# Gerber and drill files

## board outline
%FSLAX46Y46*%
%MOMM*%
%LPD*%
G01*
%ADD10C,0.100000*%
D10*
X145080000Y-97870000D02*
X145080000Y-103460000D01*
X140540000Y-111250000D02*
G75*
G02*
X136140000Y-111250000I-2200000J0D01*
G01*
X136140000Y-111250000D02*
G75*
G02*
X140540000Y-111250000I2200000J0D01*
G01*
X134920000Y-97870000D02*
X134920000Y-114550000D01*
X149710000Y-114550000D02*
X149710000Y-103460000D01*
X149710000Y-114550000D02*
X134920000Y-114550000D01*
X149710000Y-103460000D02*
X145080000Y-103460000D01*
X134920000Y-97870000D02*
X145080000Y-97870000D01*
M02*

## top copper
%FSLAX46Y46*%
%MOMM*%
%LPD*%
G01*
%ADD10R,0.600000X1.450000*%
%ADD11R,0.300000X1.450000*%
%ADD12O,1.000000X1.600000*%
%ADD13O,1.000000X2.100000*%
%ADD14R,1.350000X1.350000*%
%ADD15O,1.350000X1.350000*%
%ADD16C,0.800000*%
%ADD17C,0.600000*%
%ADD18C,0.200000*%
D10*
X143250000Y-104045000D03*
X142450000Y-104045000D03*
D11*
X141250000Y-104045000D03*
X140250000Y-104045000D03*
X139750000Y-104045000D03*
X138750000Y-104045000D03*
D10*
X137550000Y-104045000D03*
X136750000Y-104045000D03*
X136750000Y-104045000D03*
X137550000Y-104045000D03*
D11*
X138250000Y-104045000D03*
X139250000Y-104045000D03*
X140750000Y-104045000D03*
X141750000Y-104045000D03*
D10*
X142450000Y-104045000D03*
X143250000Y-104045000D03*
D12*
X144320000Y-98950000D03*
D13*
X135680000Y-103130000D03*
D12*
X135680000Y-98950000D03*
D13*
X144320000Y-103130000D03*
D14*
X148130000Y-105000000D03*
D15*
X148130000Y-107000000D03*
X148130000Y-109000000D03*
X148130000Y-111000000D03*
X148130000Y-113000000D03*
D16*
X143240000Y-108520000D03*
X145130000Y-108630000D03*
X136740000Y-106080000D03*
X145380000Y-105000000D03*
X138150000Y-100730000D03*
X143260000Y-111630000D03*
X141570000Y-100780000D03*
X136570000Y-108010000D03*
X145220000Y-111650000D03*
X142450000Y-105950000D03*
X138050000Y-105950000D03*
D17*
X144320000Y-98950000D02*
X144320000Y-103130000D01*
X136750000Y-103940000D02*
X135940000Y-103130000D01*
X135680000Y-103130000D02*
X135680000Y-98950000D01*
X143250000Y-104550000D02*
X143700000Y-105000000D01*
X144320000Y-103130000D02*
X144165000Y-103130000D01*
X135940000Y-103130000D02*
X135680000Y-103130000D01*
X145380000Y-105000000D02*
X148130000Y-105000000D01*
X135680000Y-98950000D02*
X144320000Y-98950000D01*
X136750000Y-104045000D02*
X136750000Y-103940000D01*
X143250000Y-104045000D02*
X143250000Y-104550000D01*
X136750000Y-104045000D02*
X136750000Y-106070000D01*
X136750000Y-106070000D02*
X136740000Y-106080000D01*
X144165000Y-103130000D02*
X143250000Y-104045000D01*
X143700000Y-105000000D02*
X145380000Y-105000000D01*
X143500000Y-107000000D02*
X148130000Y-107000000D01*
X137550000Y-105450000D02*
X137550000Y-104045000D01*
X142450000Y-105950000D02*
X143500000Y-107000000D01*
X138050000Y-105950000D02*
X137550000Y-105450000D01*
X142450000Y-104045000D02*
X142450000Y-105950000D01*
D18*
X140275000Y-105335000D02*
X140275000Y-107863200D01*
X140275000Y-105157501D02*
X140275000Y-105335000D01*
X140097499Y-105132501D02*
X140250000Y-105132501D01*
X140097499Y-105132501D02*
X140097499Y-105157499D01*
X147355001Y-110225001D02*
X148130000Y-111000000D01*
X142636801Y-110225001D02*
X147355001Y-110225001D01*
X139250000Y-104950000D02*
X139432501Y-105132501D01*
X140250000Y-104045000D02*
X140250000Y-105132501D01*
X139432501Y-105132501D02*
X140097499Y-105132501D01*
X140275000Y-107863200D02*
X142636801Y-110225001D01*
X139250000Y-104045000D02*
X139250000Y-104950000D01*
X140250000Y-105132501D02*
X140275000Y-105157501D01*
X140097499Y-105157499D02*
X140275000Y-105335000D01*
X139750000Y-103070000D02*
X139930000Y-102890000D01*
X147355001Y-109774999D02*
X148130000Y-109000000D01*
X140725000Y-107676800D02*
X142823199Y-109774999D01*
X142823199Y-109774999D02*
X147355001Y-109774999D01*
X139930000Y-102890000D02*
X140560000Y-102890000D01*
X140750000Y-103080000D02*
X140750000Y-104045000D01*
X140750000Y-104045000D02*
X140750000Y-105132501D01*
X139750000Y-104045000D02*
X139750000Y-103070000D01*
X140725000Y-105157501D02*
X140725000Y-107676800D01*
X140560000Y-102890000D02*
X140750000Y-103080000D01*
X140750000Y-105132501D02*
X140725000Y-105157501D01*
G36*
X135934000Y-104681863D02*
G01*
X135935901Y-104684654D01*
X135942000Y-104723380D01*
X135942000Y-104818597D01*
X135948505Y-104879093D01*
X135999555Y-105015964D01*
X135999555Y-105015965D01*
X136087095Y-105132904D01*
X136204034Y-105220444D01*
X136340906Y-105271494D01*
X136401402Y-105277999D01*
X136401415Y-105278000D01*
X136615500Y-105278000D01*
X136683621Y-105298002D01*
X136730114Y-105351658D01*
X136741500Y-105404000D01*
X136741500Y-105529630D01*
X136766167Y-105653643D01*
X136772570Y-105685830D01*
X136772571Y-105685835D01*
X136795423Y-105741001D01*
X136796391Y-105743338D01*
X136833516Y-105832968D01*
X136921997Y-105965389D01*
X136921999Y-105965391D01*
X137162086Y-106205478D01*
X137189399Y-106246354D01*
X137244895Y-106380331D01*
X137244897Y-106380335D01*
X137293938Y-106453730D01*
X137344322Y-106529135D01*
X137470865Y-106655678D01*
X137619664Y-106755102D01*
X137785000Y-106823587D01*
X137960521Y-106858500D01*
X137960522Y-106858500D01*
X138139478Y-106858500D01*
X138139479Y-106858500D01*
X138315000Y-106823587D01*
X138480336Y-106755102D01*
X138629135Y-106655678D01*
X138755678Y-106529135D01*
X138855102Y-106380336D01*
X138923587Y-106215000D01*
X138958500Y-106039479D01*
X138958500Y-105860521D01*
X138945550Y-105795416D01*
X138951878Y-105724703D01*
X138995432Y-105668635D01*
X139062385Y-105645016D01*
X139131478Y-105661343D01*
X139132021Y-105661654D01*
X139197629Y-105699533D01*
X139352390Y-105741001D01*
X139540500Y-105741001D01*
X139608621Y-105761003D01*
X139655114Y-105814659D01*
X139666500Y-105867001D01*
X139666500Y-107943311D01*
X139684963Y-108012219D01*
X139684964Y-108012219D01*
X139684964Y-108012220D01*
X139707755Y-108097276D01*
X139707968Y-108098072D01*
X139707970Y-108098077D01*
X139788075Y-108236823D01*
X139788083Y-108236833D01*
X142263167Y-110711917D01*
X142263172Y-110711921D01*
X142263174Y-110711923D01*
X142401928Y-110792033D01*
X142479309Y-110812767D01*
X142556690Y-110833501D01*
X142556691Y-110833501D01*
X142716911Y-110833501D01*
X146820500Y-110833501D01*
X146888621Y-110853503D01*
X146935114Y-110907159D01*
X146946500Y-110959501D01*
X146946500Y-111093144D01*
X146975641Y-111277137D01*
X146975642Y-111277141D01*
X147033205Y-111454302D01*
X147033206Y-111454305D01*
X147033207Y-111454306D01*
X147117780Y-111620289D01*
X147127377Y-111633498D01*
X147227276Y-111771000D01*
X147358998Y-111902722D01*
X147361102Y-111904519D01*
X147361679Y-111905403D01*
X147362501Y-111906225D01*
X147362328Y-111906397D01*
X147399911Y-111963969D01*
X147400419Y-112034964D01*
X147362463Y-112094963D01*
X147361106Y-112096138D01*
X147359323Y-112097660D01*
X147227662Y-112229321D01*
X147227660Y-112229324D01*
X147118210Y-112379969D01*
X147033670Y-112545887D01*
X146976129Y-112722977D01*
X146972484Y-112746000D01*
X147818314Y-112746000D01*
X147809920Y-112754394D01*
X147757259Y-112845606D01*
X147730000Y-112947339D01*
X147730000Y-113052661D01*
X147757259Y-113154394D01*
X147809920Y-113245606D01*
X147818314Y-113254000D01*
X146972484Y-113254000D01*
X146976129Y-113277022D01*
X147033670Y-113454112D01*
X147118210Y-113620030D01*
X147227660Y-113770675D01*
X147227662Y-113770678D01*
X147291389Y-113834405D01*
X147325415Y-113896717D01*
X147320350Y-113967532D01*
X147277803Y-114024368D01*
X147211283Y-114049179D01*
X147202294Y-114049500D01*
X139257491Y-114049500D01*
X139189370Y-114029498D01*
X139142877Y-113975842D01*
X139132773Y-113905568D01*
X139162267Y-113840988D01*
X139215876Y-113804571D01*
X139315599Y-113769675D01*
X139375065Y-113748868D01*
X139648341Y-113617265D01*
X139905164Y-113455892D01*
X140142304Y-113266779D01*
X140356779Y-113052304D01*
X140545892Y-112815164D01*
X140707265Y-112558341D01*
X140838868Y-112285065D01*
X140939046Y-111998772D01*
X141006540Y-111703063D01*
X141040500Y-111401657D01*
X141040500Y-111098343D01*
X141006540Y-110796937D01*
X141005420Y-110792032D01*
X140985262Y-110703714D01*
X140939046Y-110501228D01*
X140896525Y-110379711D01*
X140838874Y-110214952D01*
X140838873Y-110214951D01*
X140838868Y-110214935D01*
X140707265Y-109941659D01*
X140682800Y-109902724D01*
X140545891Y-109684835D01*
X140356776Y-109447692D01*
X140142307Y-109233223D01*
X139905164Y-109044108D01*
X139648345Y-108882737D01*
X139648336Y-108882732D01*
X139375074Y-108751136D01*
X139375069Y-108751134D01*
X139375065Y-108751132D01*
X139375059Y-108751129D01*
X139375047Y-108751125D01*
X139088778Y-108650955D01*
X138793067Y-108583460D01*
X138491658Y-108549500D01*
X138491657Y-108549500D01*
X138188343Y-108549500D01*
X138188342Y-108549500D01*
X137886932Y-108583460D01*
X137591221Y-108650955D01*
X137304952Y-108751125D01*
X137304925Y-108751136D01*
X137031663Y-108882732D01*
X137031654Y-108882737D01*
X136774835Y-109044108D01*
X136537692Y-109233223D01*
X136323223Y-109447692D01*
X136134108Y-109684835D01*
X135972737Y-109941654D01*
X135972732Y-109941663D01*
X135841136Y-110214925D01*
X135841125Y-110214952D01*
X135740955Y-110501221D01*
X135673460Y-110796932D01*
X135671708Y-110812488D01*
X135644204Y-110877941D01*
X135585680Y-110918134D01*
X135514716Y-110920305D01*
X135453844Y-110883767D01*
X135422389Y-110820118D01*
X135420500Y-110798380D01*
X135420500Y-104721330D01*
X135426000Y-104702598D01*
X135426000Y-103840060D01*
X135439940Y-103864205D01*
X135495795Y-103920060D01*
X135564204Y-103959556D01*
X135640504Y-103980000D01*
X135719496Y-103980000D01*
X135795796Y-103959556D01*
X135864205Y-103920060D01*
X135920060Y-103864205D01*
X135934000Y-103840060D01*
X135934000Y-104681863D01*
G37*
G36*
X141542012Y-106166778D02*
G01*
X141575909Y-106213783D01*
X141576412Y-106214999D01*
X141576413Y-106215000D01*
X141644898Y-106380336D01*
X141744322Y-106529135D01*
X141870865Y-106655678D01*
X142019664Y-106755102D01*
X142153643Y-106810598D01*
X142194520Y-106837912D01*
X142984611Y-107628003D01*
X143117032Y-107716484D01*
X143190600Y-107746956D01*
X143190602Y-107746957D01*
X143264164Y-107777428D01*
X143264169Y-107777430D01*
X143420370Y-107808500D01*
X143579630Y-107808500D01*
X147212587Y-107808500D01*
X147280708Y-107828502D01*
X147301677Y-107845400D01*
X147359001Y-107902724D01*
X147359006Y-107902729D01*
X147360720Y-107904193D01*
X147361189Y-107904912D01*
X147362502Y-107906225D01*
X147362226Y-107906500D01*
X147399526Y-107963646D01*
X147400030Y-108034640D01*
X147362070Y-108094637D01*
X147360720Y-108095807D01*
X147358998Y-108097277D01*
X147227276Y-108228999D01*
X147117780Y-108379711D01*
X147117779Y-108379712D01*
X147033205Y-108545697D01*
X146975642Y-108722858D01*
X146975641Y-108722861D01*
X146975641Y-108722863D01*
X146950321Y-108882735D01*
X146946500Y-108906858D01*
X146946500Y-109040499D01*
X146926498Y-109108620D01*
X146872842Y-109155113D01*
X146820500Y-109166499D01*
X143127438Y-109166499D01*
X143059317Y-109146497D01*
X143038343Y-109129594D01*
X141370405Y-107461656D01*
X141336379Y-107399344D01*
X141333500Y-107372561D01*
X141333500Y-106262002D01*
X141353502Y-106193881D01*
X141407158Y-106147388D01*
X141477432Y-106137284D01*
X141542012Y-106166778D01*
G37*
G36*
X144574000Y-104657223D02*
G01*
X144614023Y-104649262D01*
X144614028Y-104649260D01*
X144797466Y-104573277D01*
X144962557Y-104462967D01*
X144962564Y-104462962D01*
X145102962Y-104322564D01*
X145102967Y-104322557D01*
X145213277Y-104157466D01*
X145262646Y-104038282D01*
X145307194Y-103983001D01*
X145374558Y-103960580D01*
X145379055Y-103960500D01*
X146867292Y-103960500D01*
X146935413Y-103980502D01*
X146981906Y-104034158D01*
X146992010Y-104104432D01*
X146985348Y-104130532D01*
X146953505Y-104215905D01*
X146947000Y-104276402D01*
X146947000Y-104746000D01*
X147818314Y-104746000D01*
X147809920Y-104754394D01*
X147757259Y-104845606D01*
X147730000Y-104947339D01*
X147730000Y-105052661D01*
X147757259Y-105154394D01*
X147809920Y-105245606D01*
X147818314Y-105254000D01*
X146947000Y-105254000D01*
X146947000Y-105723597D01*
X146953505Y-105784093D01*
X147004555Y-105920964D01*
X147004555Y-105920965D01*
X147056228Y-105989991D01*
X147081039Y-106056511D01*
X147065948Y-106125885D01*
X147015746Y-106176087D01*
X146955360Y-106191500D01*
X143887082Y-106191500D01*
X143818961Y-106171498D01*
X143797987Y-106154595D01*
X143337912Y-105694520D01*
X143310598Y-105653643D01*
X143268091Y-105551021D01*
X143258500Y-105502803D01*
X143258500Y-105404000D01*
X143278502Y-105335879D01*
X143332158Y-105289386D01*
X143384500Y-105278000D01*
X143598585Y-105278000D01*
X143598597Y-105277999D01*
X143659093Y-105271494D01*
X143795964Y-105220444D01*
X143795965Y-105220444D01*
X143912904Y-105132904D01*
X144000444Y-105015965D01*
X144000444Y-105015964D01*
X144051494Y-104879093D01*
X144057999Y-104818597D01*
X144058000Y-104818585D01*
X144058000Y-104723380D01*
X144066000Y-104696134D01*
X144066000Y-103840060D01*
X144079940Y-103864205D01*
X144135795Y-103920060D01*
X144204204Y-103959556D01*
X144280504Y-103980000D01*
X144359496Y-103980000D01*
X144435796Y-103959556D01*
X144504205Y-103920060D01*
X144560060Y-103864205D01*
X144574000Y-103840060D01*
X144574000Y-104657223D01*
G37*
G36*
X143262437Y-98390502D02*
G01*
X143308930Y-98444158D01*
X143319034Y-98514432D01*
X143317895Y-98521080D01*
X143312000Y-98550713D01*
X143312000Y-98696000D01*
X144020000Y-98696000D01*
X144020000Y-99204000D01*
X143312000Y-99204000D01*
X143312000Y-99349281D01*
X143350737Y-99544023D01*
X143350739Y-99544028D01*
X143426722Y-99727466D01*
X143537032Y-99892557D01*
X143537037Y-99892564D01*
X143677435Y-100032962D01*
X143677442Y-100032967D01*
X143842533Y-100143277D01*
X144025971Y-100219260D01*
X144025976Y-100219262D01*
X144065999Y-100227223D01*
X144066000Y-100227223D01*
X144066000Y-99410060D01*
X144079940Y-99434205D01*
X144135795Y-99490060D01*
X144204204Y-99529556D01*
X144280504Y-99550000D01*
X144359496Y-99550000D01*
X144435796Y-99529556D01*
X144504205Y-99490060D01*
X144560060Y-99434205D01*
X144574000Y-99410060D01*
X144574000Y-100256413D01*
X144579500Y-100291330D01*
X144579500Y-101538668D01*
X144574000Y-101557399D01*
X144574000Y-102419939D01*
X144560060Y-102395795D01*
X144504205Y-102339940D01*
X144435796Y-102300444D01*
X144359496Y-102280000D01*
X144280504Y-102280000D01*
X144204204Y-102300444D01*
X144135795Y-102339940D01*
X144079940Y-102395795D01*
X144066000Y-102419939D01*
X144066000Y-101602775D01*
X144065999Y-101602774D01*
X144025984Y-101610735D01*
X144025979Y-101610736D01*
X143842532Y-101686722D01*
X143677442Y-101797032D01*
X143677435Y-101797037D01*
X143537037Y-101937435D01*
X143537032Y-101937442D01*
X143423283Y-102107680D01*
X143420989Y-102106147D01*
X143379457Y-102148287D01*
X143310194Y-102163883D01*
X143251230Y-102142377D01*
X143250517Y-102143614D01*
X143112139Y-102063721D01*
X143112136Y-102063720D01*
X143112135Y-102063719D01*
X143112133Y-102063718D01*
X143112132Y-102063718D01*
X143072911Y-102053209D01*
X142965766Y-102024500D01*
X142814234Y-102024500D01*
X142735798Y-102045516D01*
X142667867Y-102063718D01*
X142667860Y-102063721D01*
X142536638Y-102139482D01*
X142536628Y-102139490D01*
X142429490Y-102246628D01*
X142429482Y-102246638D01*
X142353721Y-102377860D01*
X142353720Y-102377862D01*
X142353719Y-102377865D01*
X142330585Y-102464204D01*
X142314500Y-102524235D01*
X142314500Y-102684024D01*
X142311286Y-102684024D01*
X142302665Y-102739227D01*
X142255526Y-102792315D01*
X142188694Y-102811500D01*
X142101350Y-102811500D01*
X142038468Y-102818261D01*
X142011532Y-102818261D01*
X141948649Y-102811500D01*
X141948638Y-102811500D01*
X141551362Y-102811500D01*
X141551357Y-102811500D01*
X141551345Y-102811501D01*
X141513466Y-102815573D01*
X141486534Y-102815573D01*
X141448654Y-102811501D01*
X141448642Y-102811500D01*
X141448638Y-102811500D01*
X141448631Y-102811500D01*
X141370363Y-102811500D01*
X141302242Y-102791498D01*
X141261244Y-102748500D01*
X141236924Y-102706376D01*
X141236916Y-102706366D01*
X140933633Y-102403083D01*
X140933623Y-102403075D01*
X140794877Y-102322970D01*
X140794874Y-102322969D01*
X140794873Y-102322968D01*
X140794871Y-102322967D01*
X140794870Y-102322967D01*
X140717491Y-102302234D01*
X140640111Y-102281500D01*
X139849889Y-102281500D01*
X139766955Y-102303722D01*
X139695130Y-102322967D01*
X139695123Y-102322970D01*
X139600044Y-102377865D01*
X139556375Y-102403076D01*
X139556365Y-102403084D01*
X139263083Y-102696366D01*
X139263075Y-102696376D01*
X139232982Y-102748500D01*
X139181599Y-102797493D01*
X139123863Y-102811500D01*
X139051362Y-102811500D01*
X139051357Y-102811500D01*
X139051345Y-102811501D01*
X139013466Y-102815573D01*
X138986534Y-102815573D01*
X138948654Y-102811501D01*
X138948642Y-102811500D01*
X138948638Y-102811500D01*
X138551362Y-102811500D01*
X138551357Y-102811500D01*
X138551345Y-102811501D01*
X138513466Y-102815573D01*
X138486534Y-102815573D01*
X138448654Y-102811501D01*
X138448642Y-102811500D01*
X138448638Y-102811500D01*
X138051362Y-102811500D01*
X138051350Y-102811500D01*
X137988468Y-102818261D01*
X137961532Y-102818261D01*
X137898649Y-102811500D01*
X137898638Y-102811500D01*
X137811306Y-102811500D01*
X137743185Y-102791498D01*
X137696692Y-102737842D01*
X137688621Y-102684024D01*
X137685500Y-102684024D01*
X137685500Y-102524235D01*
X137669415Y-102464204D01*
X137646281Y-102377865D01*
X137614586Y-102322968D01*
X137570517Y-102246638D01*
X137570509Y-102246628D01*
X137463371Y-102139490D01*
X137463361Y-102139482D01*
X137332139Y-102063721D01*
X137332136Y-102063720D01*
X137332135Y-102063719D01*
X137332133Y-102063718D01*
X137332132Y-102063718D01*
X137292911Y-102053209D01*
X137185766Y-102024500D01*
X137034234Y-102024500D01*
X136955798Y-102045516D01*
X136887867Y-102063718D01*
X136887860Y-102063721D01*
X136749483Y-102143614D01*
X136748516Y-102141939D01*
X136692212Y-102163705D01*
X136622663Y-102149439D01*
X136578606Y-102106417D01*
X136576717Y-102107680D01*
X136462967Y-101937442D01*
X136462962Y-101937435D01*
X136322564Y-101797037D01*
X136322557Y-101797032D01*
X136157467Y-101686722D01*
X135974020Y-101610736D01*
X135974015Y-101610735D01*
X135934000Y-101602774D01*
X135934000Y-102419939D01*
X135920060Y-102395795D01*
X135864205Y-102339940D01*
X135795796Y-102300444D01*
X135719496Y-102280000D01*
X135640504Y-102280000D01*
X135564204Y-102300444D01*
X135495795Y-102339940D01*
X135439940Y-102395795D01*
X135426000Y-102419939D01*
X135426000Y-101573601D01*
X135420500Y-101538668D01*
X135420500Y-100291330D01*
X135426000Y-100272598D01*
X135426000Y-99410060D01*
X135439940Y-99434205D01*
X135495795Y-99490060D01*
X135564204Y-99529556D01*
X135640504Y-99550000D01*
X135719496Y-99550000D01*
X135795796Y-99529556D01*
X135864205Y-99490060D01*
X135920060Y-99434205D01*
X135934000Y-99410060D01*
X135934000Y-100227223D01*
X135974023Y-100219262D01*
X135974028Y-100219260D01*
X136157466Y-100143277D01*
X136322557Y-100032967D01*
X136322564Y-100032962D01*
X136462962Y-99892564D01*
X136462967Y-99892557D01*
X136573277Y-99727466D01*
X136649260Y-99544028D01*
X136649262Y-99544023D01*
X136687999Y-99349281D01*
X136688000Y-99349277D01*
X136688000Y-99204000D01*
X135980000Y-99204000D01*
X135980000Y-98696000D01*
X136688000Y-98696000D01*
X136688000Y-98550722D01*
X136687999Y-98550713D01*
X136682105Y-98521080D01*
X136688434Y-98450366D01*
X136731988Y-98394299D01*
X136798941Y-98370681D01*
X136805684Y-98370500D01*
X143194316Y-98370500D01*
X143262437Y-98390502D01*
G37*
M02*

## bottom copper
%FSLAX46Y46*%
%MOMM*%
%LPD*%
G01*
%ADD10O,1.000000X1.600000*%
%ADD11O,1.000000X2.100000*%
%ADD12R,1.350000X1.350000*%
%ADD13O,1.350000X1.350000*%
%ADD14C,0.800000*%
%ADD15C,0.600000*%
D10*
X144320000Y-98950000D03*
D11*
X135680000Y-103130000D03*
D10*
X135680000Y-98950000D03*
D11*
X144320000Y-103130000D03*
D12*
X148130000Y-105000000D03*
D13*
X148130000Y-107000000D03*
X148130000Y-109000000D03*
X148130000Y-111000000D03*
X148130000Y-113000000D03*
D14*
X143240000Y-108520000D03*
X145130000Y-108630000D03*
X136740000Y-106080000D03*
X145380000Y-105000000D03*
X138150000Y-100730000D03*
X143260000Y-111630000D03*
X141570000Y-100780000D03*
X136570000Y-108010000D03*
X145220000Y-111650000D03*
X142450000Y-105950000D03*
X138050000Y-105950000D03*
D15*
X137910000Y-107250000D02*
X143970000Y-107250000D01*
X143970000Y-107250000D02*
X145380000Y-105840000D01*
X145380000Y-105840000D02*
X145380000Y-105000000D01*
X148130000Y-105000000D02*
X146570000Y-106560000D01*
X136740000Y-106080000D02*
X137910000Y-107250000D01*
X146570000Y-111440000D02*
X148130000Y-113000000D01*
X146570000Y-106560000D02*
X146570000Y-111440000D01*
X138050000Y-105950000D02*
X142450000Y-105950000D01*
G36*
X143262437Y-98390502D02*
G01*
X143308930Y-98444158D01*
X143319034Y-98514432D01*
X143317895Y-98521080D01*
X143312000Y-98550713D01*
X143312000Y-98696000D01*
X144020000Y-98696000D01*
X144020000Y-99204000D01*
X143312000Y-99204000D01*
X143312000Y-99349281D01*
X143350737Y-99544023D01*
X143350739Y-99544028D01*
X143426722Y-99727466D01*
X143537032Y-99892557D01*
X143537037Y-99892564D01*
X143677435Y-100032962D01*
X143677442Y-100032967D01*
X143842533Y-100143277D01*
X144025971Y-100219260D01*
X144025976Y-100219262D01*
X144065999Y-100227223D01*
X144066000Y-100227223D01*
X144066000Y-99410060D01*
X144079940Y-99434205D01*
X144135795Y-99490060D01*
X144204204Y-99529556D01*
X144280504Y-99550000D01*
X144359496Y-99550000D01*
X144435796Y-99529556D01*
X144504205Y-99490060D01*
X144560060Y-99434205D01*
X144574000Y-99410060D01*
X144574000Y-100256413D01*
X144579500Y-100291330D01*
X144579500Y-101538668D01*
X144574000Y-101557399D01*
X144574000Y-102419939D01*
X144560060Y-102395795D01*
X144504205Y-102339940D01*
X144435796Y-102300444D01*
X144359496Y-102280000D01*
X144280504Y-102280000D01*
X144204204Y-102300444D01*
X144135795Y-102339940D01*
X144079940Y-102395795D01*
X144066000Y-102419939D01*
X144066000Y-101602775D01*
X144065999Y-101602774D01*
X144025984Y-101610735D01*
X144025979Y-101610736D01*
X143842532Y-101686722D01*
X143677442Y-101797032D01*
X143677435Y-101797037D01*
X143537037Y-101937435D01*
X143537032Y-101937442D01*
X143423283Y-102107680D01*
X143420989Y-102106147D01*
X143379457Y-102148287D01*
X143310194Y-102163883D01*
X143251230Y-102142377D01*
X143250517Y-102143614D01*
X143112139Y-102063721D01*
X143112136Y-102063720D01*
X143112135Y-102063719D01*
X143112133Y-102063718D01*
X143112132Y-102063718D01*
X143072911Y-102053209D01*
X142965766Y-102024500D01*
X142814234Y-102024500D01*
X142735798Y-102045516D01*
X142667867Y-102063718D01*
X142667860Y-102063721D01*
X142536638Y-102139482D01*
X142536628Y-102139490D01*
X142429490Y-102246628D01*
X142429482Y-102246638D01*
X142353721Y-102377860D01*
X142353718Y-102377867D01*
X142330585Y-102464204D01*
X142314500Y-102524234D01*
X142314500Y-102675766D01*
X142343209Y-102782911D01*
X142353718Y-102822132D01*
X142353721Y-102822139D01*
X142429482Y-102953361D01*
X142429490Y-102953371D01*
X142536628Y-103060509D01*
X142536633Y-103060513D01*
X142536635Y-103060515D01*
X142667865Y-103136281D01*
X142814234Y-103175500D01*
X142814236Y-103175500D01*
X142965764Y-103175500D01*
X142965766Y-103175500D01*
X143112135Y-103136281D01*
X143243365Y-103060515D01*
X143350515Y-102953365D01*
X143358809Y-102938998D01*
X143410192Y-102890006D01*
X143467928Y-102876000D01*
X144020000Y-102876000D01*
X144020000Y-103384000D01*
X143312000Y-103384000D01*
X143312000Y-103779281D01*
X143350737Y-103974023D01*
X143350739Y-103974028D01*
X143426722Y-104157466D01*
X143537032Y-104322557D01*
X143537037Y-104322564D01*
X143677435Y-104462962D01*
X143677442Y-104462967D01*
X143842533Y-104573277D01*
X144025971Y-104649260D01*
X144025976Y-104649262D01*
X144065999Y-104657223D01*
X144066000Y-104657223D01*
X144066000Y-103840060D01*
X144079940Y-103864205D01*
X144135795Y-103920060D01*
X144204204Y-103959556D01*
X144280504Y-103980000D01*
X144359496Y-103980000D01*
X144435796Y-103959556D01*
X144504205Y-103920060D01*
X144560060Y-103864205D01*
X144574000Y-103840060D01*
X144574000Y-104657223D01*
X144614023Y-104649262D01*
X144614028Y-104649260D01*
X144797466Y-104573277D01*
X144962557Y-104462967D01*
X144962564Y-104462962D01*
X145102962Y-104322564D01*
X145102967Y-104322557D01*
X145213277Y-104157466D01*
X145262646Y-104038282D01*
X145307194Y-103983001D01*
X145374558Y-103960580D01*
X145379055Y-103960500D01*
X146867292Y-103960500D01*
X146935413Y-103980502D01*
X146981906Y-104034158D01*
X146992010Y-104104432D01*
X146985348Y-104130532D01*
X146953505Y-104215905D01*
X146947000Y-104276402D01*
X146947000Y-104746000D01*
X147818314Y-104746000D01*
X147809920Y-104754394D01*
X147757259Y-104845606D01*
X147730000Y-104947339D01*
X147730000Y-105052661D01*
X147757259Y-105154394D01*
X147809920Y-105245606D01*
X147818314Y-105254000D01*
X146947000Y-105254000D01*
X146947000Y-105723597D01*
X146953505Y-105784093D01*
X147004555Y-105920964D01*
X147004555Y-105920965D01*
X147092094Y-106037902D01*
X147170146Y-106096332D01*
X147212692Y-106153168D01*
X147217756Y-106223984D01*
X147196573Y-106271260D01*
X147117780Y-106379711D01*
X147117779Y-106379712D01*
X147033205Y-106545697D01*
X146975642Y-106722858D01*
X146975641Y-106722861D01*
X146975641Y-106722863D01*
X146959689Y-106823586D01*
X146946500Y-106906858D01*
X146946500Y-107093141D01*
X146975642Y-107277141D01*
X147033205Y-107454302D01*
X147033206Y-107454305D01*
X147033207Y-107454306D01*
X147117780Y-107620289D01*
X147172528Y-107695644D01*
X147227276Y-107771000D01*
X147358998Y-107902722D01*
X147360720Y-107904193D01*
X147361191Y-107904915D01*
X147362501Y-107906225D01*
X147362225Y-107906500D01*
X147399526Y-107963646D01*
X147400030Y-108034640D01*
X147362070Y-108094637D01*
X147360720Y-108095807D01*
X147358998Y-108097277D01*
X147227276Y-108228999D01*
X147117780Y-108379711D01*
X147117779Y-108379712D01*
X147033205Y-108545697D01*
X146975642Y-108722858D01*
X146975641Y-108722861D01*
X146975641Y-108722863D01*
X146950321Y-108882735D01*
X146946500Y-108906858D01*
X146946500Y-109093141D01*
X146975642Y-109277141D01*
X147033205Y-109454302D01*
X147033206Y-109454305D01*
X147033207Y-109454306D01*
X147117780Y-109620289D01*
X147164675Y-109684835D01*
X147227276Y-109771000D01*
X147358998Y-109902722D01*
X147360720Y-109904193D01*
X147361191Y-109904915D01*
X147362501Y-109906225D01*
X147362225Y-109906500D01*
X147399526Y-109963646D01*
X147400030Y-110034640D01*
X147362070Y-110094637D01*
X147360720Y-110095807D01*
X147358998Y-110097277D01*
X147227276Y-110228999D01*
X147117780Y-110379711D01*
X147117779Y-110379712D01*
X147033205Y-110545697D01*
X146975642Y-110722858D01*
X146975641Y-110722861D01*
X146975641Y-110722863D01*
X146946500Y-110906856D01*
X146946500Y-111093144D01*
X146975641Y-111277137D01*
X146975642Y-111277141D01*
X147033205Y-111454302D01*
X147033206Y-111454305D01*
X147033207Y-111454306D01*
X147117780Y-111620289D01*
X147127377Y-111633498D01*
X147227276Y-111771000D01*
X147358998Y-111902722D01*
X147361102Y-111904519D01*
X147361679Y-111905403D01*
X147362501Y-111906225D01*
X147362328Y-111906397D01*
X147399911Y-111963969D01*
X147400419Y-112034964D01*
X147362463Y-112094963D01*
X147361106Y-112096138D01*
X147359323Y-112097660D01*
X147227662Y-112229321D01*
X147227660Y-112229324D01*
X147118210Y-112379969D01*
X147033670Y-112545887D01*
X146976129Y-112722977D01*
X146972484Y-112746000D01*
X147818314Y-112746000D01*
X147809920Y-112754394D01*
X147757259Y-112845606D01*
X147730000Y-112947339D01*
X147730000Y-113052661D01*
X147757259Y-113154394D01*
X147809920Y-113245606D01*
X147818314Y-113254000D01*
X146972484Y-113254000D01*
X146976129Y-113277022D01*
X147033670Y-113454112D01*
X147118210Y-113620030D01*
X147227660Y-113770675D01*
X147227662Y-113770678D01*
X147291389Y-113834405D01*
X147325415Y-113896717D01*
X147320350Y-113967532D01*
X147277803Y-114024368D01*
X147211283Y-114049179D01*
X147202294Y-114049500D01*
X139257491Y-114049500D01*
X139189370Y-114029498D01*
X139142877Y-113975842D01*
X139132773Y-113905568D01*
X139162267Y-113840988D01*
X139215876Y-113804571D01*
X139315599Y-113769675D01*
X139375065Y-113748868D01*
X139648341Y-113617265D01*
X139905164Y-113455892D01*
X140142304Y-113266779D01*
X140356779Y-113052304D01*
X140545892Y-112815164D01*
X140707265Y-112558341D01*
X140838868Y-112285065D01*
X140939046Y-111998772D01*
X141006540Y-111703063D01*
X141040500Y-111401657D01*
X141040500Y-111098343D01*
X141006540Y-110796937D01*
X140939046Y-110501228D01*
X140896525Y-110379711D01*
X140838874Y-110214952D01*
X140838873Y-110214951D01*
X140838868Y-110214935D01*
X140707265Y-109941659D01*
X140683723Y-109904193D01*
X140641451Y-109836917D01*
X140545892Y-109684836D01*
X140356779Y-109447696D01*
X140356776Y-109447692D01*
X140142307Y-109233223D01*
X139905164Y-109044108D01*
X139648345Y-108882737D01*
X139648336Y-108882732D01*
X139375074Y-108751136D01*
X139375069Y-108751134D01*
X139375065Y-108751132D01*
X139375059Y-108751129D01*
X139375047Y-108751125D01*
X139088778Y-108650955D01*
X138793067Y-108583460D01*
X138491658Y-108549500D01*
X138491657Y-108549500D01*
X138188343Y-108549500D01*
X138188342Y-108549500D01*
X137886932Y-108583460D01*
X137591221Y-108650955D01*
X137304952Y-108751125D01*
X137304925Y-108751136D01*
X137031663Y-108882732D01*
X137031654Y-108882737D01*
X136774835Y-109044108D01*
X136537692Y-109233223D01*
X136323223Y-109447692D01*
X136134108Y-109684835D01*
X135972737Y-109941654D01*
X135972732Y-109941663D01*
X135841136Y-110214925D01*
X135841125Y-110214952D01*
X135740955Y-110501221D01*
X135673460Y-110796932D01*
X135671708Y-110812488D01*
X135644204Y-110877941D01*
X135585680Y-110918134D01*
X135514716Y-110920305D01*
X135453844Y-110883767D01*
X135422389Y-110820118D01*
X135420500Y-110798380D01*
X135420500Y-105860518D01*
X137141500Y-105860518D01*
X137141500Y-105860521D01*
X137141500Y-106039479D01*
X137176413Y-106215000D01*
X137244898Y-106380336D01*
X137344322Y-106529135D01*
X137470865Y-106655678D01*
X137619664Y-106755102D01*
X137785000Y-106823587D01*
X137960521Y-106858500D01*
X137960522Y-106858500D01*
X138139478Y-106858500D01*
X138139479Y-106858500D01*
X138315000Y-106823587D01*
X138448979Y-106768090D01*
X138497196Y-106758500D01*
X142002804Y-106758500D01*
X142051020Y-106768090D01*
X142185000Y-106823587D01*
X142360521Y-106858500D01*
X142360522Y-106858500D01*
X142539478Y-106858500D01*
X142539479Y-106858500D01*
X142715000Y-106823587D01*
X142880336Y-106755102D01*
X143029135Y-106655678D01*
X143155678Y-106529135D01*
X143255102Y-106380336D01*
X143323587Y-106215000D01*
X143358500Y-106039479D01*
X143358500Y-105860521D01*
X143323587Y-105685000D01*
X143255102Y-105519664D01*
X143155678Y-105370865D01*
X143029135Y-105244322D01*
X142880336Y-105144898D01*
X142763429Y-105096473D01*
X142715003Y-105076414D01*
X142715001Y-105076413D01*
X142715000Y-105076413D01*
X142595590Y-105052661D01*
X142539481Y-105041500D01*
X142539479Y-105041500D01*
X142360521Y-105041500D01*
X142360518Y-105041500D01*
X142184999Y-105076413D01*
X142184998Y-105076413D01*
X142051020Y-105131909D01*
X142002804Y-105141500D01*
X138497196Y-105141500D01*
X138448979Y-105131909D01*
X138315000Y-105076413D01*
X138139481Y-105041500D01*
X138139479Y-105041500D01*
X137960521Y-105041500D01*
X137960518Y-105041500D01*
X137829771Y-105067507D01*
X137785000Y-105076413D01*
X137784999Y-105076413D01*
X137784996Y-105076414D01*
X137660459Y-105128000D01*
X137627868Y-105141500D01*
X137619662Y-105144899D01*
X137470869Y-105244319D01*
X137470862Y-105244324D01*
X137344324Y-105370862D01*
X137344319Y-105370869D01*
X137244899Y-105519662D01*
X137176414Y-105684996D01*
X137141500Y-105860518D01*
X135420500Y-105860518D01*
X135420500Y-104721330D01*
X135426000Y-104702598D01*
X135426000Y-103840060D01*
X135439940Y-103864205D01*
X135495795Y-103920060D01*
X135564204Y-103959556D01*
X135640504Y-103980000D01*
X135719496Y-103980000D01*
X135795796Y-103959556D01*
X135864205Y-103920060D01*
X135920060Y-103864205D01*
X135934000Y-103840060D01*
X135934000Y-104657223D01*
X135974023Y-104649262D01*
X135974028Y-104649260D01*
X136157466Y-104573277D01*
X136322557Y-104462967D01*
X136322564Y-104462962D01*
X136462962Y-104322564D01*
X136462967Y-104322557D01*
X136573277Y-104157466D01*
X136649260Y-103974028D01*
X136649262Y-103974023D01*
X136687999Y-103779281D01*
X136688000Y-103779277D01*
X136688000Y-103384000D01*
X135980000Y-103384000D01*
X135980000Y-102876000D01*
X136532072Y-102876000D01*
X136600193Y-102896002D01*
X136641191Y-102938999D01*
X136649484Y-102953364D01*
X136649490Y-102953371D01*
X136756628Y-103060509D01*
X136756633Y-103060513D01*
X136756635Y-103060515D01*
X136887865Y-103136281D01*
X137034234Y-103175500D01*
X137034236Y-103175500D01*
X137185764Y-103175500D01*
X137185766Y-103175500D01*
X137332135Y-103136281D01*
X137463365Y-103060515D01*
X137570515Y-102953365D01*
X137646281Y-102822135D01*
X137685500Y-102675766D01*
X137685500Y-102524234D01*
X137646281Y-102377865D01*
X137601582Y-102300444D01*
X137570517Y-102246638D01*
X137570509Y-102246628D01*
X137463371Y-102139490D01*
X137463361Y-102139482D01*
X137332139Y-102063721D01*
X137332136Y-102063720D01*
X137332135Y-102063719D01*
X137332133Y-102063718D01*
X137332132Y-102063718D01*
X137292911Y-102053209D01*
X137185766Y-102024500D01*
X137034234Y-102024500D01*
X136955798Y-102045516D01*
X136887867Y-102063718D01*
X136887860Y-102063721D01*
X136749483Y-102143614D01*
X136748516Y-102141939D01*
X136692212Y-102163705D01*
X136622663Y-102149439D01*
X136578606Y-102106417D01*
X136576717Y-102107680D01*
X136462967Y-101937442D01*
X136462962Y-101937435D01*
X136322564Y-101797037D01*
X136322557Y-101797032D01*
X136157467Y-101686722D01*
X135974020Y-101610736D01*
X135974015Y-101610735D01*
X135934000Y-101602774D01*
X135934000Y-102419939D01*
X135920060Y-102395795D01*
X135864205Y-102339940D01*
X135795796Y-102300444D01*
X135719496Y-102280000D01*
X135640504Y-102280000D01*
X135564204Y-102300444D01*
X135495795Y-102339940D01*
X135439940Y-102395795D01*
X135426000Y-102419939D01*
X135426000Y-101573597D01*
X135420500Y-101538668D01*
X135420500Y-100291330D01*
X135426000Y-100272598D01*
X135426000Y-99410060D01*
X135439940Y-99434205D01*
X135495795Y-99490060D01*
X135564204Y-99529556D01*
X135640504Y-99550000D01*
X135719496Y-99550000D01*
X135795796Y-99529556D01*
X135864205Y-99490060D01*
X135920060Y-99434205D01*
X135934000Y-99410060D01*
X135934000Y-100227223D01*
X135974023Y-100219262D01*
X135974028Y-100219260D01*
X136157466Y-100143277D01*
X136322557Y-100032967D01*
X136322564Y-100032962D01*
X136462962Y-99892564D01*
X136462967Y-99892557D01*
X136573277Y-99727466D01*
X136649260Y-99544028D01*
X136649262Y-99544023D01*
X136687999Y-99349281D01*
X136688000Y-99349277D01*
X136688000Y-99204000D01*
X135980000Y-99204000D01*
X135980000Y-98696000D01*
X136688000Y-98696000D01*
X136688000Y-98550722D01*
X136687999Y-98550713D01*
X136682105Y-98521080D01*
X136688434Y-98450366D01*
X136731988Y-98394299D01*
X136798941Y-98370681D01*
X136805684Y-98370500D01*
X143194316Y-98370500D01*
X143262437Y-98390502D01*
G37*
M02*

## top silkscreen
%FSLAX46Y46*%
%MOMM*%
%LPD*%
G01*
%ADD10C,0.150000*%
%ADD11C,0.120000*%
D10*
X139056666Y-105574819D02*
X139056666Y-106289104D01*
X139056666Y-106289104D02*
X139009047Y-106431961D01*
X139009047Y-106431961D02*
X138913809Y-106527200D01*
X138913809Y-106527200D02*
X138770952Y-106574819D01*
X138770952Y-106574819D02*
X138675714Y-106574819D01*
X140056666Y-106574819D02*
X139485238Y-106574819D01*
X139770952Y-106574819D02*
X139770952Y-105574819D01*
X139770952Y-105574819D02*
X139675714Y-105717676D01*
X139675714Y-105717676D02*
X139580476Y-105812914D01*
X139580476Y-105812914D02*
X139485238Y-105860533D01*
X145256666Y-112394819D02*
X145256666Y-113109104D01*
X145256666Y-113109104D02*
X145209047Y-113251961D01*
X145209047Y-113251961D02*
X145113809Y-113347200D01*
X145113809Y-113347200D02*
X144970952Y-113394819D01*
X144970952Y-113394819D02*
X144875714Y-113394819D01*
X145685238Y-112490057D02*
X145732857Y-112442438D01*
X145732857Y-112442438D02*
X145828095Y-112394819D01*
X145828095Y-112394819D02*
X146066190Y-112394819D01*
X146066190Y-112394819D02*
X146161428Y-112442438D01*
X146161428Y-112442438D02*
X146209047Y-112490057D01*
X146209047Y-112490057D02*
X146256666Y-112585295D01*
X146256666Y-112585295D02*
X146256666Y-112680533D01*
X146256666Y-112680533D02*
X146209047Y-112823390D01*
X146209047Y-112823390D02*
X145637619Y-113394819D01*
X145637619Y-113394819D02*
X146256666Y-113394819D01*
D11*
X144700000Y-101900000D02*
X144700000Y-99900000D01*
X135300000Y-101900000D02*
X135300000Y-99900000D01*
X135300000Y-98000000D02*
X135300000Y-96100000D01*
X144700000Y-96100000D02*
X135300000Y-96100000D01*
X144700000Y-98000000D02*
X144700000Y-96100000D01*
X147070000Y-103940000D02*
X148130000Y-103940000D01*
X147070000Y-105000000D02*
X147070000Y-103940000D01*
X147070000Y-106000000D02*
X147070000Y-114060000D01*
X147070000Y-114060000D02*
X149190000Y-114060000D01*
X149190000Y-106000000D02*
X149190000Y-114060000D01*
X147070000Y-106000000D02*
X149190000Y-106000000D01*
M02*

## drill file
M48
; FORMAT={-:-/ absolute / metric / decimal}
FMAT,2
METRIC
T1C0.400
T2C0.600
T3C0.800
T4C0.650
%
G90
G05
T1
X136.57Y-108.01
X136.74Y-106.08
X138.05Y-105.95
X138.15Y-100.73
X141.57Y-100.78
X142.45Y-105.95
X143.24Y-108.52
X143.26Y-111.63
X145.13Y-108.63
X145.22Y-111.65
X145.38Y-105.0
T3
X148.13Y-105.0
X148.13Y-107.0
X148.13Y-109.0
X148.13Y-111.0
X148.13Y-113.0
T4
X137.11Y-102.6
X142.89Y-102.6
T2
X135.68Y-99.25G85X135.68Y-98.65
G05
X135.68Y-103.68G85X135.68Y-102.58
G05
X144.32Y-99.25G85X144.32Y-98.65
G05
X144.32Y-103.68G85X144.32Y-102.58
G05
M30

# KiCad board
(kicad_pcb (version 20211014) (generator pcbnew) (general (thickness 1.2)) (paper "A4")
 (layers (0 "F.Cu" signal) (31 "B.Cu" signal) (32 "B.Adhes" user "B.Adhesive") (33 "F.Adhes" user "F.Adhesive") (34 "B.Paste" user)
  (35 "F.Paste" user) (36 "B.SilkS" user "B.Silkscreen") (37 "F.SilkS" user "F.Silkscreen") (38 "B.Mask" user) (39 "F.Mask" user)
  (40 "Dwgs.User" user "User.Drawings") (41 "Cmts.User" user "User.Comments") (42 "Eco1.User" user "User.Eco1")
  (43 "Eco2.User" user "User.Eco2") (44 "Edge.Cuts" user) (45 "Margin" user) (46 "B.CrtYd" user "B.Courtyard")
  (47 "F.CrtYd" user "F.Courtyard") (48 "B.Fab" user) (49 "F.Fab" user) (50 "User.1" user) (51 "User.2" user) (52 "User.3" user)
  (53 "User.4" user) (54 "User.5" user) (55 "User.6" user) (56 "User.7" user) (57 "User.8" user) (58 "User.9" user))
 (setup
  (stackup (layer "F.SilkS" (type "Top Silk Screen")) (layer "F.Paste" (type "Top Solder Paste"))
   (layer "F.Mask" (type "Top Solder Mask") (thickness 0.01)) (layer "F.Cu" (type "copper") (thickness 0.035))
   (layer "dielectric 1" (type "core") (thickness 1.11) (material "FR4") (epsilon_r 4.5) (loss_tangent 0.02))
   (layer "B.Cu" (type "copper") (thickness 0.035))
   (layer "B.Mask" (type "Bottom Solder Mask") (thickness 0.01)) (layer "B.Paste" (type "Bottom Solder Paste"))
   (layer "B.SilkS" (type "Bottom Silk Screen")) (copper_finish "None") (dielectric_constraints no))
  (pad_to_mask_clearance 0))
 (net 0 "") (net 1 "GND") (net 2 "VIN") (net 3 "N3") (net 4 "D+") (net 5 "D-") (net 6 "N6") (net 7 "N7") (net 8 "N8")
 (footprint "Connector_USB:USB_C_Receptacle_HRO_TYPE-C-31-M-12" (layer "F.Cu") (at 140 100 180)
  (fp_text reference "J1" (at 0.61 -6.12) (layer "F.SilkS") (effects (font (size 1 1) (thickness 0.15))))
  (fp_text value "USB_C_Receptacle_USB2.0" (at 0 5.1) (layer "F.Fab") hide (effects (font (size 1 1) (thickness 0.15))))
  (fp_line (start -4.7 -1.9) (end -4.7 0.1) (layer "F.SilkS") (width 0.12))
  (fp_line (start 4.7 -1.9) (end 4.7 0.1) (layer "F.SilkS") (width 0.12))
  (fp_line (start 4.7 2) (end 4.7 3.9) (layer "F.SilkS") (width 0.12))
  (fp_line (start -4.7 3.9) (end 4.7 3.9) (layer "F.SilkS") (width 0.12))
  (fp_line (start -4.7 2) (end -4.7 3.9) (layer "F.SilkS") (width 0.12))
  (pad "" np_thru_hole circle (at -2.89 -2.6 180) (size 0.65 0.65) (drill 0.65) (layers *.Cu *.Mask))
  (pad "" np_thru_hole circle (at 2.89 -2.6 180) (size 0.65 0.65) (drill 0.65) (layers *.Cu *.Mask))
  (pad "A1" smd rect (at -3.25 -4.045 180) (size 0.6 1.45) (layers "F.Cu" "F.Paste" "F.Mask") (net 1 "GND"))
  (pad "A4" smd rect (at -2.45 -4.045 180) (size 0.6 1.45) (layers "F.Cu" "F.Paste" "F.Mask") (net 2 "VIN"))
  (pad "A5" smd rect (at -1.25 -4.045 180) (size 0.3 1.45) (layers "F.Cu" "F.Paste" "F.Mask") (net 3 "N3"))
  (pad "A6" smd rect (at -0.25 -4.045 180) (size 0.3 1.45) (layers "F.Cu" "F.Paste" "F.Mask") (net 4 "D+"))
  (pad "A7" smd rect (at 0.25 -4.045 180) (size 0.3 1.45) (layers "F.Cu" "F.Paste" "F.Mask") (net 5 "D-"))
  (pad "A8" smd rect (at 1.25 -4.045 180) (size 0.3 1.45) (layers "F.Cu" "F.Paste" "F.Mask") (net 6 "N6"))
  (pad "A9" smd rect (at 2.45 -4.045 180) (size 0.6 1.45) (layers "F.Cu" "F.Paste" "F.Mask") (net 2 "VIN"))
  (pad "A12" smd rect (at 3.25 -4.045 180) (size 0.6 1.45) (layers "F.Cu" "F.Paste" "F.Mask") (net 1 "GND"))
  (pad "B1" smd rect (at 3.25 -4.045 180) (size 0.6 1.45) (layers "F.Cu" "F.Paste" "F.Mask") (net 1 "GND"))
  (pad "B4" smd rect (at 2.45 -4.045 180) (size 0.6 1.45) (layers "F.Cu" "F.Paste" "F.Mask") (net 2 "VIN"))
  (pad "B5" smd rect (at 1.75 -4.045 180) (size 0.3 1.45) (layers "F.Cu" "F.Paste" "F.Mask") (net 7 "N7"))
  (pad "B6" smd rect (at 0.75 -4.045 180) (size 0.3 1.45) (layers "F.Cu" "F.Paste" "F.Mask") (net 4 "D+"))
  (pad "B7" smd rect (at -0.75 -4.045 180) (size 0.3 1.45) (layers "F.Cu" "F.Paste" "F.Mask") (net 5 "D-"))
  (pad "B8" smd rect (at -1.75 -4.045 180) (size 0.3 1.45) (layers "F.Cu" "F.Paste" "F.Mask") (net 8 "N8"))
  (pad "B9" smd rect (at -2.45 -4.045 180) (size 0.6 1.45) (layers "F.Cu" "F.Paste" "F.Mask") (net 2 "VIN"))
  (pad "B12" smd rect (at -3.25 -4.045 180) (size 0.6 1.45) (layers "F.Cu" "F.Paste" "F.Mask") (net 1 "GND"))
  (pad "S1" thru_hole oval (at -4.32 1.05 180) (size 1 1.6) (drill oval 0.6 1.2) (layers *.Cu *.Mask) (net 1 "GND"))
  (pad "S1" thru_hole oval (at 4.32 -3.13 180) (size 1 2.1) (drill oval 0.6 1.7) (layers *.Cu *.Mask) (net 1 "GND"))
  (pad "S1" thru_hole oval (at 4.32 1.05 180) (size 1 1.6) (drill oval 0.6 1.2) (layers *.Cu *.Mask) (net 1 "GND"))
  (pad "S1" thru_hole oval (at -4.32 -3.13 180) (size 1 2.1) (drill oval 0.6 1.7) (layers *.Cu *.Mask) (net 1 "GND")))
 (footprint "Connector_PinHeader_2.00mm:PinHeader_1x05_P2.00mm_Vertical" (layer "F.Cu") (at 148.13 105)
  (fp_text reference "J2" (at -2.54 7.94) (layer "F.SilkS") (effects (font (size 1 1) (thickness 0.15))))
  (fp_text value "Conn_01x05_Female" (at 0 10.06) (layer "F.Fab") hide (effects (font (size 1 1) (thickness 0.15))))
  (fp_line (start -1.06 -1.06) (end 0 -1.06) (layer "F.SilkS") (width 0.12))
  (fp_line (start -1.06 0) (end -1.06 -1.06) (layer "F.SilkS") (width 0.12))
  (fp_line (start -1.06 1) (end -1.06 9.06) (layer "F.SilkS") (width 0.12))
  (fp_line (start -1.06 9.06) (end 1.06 9.06) (layer "F.SilkS") (width 0.12))
  (fp_line (start 1.06 1) (end 1.06 9.06) (layer "F.SilkS") (width 0.12))
  (fp_line (start -1.06 1) (end 1.06 1) (layer "F.SilkS") (width 0.12))
  (pad "1" thru_hole rect (at 0 0) (size 1.35 1.35) (drill 0.8) (layers *.Cu *.Mask) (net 1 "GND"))
  (pad "2" thru_hole oval (at 0 2) (size 1.35 1.35) (drill 0.8) (layers *.Cu *.Mask) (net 2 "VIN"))
  (pad "3" thru_hole oval (at 0 4) (size 1.35 1.35) (drill 0.8) (layers *.Cu *.Mask) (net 5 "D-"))
  (pad "4" thru_hole oval (at 0 6) (size 1.35 1.35) (drill 0.8) (layers *.Cu *.Mask) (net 4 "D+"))
  (pad "5" thru_hole oval (at 0 8) (size 1.35 1.35) (drill 0.8) (layers *.Cu *.Mask) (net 1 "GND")))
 (gr_line (start 145.08 97.87) (end 145.08 103.46) (layer "Edge.Cuts") (width 0.1))
 (gr_circle (center 138.34 111.25) (end 140.54 111.25) (layer "Edge.Cuts") (width 0.1) (fill none))
 (gr_line (start 134.92 97.87) (end 134.92 114.55) (layer "Edge.Cuts") (width 0.1))
 (gr_line (start 149.71 114.55) (end 149.71 103.46) (layer "Edge.Cuts") (width 0.1))
 (gr_line (start 149.71 114.55) (end 134.92 114.55) (layer "Edge.Cuts") (width 0.1))
 (gr_line (start 149.71 103.46) (end 145.08 103.46) (layer "Edge.Cuts") (width 0.1))
 (gr_line (start 134.92 97.87) (end 145.08 97.87) (layer "Edge.Cuts") (width 0.1))
 (segment (start 144.32 98.95) (end 144.32 103.13) (width 0.6) (layer "F.Cu") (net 1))
 (segment (start 136.75 103.94) (end 135.94 103.13) (width 0.6) (layer "F.Cu") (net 1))
 (segment (start 135.68 103.13) (end 135.68 98.95) (width 0.6) (layer "F.Cu") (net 1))
 (segment (start 143.25 104.55) (end 143.7 105) (width 0.6) (layer "F.Cu") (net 1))
 (segment (start 144.32 103.13) (end 144.165 103.13) (width 0.6) (layer "F.Cu") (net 1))
 (segment (start 135.94 103.13) (end 135.68 103.13) (width 0.6) (layer "F.Cu") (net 1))
 (segment (start 145.38 105) (end 148.13 105) (width 0.6) (layer "F.Cu") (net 1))
 (segment (start 135.68 98.95) (end 144.32 98.95) (width 0.6) (layer "F.Cu") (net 1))
 (segment (start 136.75 104.045) (end 136.75 103.94) (width 0.6) (layer "F.Cu") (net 1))
 (segment (start 143.25 104.045) (end 143.25 104.55) (width 0.6) (layer "F.Cu") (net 1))
 (segment (start 136.75 104.045) (end 136.75 106.07) (width 0.6) (layer "F.Cu") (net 1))
 (segment (start 136.75 106.07) (end 136.74 106.08) (width 0.6) (layer "F.Cu") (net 1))
 (segment (start 144.165 103.13) (end 143.25 104.045) (width 0.6) (layer "F.Cu") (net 1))
 (segment (start 143.7 105) (end 145.38 105) (width 0.6) (layer "F.Cu") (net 1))
 (via (at 143.24 108.52) (size 0.8) (drill 0.4) (layers "F.Cu" "B.Cu") (free) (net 1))
 (via (at 145.13 108.63) (size 0.8) (drill 0.4) (layers "F.Cu" "B.Cu") (free) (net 1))
 (via (at 136.74 106.08) (size 0.8) (drill 0.4) (layers "F.Cu" "B.Cu") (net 1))
 (via (at 145.38 105) (size 0.8) (drill 0.4) (layers "F.Cu" "B.Cu") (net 1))
 (via (at 138.15 100.73) (size 0.8) (drill 0.4) (layers "F.Cu" "B.Cu") (free) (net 1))
 (via (at 143.26 111.63) (size 0.8) (drill 0.4) (layers "F.Cu" "B.Cu") (free) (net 1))
 (via (at 141.57 100.78) (size 0.8) (drill 0.4) (layers "F.Cu" "B.Cu") (free) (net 1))
 (via (at 136.57 108.01) (size 0.8) (drill 0.4) (layers "F.Cu" "B.Cu") (free) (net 1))
 (via (at 145.22 111.65) (size 0.8) (drill 0.4) (layers "F.Cu" "B.Cu") (free) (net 1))
 (segment (start 137.91 107.25) (end 143.97 107.25) (width 0.6) (layer "B.Cu") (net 1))
 (segment (start 143.97 107.25) (end 145.38 105.84) (width 0.6) (layer "B.Cu") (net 1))
 (segment (start 145.38 105.84) (end 145.38 105) (width 0.6) (layer "B.Cu") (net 1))
 (segment (start 148.13 105) (end 146.57 106.56) (width 0.6) (layer "B.Cu") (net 1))
 (segment (start 136.74 106.08) (end 137.91 107.25) (width 0.6) (layer "B.Cu") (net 1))
 (segment (start 146.57 111.44) (end 148.13 113) (width 0.6) (layer "B.Cu") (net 1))
 (segment (start 146.57 106.56) (end 146.57 111.44) (width 0.6) (layer "B.Cu") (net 1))
 (segment (start 143.5 107) (end 148.13 107) (width 0.6) (layer "F.Cu") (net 2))
 (segment (start 137.55 105.45) (end 137.55 104.045) (width 0.6) (layer "F.Cu") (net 2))
 (segment (start 142.45 105.95) (end 143.5 107) (width 0.6) (layer "F.Cu") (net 2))
 (segment (start 138.05 105.95) (end 137.55 105.45) (width 0.6) (layer "F.Cu") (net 2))
 (segment (start 142.45 104.045) (end 142.45 105.95) (width 0.6) (layer "F.Cu") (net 2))
 (via (at 142.45 105.95) (size 0.8) (drill 0.4) (layers "F.Cu" "B.Cu") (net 2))
 (via (at 138.05 105.95) (size 0.8) (drill 0.4) (layers "F.Cu" "B.Cu") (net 2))
 (segment (start 138.05 105.95) (end 142.45 105.95) (width 0.6) (layer "B.Cu") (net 2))
 (segment (start 140.275 105.335) (end 140.275 107.8632) (width 0.2) (layer "F.Cu") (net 4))
 (segment (start 140.275 105.157501) (end 140.275 105.335) (width 0.2) (layer "F.Cu") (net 4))
 (segment (start 140.097499 105.132501) (end 140.25 105.132501) (width 0.2) (layer "F.Cu") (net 4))
 (segment (start 140.097499 105.132501) (end 140.097499 105.157499) (width 0.2) (layer "F.Cu") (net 4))
 (segment (start 147.355001 110.225001) (end 148.13 111) (width 0.2) (layer "F.Cu") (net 4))
 (segment (start 142.636801 110.225001) (end 147.355001 110.225001) (width 0.2) (layer "F.Cu") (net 4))
 (segment (start 139.25 104.95) (end 139.432501 105.132501) (width 0.2) (layer "F.Cu") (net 4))
 (segment (start 140.25 104.045) (end 140.25 105.132501) (width 0.2) (layer "F.Cu") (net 4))
 (segment (start 139.432501 105.132501) (end 140.097499 105.132501) (width 0.2) (layer "F.Cu") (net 4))
 (segment (start 140.275 107.8632) (end 142.636801 110.225001) (width 0.2) (layer "F.Cu") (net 4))
 (segment (start 139.25 104.045) (end 139.25 104.95) (width 0.2) (layer "F.Cu") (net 4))
 (segment (start 140.25 105.132501) (end 140.275 105.157501) (width 0.2) (layer "F.Cu") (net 4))
 (segment (start 140.097499 105.157499) (end 140.275 105.335) (width 0.2) (layer "F.Cu") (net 4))
 (segment (start 139.75 103.07) (end 139.93 102.89) (width 0.2) (layer "F.Cu") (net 5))
 (segment (start 147.355001 109.774999) (end 148.13 109) (width 0.2) (layer "F.Cu") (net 5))
 (segment (start 140.725 107.6768) (end 142.823199 109.774999) (width 0.2) (layer "F.Cu") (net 5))
 (segment (start 142.823199 109.774999) (end 147.355001 109.774999) (width 0.2) (layer "F.Cu") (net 5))
 (segment (start 139.93 102.89) (end 140.56 102.89) (width 0.2) (layer "F.Cu") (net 5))
 (segment (start 140.75 103.08) (end 140.75 104.045) (width 0.2) (layer "F.Cu") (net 5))
 (segment (start 140.75 104.045) (end 140.75 105.132501) (width 0.2) (layer "F.Cu") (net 5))
 (segment (start 139.75 104.045) (end 139.75 103.07) (width 0.2) (layer "F.Cu") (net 5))
 (segment (start 140.725 105.157501) (end 140.725 107.6768) (width 0.2) (layer "F.Cu") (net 5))
 (segment (start 140.56 102.89) (end 140.75 103.08) (width 0.2) (layer "F.Cu") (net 5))
 (segment (start 140.75 105.132501) (end 140.725 105.157501) (width 0.2) (layer "F.Cu") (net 5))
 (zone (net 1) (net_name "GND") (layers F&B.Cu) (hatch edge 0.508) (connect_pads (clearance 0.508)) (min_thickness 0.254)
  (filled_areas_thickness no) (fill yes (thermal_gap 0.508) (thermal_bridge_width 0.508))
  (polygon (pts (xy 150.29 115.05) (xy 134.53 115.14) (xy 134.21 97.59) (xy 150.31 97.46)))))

